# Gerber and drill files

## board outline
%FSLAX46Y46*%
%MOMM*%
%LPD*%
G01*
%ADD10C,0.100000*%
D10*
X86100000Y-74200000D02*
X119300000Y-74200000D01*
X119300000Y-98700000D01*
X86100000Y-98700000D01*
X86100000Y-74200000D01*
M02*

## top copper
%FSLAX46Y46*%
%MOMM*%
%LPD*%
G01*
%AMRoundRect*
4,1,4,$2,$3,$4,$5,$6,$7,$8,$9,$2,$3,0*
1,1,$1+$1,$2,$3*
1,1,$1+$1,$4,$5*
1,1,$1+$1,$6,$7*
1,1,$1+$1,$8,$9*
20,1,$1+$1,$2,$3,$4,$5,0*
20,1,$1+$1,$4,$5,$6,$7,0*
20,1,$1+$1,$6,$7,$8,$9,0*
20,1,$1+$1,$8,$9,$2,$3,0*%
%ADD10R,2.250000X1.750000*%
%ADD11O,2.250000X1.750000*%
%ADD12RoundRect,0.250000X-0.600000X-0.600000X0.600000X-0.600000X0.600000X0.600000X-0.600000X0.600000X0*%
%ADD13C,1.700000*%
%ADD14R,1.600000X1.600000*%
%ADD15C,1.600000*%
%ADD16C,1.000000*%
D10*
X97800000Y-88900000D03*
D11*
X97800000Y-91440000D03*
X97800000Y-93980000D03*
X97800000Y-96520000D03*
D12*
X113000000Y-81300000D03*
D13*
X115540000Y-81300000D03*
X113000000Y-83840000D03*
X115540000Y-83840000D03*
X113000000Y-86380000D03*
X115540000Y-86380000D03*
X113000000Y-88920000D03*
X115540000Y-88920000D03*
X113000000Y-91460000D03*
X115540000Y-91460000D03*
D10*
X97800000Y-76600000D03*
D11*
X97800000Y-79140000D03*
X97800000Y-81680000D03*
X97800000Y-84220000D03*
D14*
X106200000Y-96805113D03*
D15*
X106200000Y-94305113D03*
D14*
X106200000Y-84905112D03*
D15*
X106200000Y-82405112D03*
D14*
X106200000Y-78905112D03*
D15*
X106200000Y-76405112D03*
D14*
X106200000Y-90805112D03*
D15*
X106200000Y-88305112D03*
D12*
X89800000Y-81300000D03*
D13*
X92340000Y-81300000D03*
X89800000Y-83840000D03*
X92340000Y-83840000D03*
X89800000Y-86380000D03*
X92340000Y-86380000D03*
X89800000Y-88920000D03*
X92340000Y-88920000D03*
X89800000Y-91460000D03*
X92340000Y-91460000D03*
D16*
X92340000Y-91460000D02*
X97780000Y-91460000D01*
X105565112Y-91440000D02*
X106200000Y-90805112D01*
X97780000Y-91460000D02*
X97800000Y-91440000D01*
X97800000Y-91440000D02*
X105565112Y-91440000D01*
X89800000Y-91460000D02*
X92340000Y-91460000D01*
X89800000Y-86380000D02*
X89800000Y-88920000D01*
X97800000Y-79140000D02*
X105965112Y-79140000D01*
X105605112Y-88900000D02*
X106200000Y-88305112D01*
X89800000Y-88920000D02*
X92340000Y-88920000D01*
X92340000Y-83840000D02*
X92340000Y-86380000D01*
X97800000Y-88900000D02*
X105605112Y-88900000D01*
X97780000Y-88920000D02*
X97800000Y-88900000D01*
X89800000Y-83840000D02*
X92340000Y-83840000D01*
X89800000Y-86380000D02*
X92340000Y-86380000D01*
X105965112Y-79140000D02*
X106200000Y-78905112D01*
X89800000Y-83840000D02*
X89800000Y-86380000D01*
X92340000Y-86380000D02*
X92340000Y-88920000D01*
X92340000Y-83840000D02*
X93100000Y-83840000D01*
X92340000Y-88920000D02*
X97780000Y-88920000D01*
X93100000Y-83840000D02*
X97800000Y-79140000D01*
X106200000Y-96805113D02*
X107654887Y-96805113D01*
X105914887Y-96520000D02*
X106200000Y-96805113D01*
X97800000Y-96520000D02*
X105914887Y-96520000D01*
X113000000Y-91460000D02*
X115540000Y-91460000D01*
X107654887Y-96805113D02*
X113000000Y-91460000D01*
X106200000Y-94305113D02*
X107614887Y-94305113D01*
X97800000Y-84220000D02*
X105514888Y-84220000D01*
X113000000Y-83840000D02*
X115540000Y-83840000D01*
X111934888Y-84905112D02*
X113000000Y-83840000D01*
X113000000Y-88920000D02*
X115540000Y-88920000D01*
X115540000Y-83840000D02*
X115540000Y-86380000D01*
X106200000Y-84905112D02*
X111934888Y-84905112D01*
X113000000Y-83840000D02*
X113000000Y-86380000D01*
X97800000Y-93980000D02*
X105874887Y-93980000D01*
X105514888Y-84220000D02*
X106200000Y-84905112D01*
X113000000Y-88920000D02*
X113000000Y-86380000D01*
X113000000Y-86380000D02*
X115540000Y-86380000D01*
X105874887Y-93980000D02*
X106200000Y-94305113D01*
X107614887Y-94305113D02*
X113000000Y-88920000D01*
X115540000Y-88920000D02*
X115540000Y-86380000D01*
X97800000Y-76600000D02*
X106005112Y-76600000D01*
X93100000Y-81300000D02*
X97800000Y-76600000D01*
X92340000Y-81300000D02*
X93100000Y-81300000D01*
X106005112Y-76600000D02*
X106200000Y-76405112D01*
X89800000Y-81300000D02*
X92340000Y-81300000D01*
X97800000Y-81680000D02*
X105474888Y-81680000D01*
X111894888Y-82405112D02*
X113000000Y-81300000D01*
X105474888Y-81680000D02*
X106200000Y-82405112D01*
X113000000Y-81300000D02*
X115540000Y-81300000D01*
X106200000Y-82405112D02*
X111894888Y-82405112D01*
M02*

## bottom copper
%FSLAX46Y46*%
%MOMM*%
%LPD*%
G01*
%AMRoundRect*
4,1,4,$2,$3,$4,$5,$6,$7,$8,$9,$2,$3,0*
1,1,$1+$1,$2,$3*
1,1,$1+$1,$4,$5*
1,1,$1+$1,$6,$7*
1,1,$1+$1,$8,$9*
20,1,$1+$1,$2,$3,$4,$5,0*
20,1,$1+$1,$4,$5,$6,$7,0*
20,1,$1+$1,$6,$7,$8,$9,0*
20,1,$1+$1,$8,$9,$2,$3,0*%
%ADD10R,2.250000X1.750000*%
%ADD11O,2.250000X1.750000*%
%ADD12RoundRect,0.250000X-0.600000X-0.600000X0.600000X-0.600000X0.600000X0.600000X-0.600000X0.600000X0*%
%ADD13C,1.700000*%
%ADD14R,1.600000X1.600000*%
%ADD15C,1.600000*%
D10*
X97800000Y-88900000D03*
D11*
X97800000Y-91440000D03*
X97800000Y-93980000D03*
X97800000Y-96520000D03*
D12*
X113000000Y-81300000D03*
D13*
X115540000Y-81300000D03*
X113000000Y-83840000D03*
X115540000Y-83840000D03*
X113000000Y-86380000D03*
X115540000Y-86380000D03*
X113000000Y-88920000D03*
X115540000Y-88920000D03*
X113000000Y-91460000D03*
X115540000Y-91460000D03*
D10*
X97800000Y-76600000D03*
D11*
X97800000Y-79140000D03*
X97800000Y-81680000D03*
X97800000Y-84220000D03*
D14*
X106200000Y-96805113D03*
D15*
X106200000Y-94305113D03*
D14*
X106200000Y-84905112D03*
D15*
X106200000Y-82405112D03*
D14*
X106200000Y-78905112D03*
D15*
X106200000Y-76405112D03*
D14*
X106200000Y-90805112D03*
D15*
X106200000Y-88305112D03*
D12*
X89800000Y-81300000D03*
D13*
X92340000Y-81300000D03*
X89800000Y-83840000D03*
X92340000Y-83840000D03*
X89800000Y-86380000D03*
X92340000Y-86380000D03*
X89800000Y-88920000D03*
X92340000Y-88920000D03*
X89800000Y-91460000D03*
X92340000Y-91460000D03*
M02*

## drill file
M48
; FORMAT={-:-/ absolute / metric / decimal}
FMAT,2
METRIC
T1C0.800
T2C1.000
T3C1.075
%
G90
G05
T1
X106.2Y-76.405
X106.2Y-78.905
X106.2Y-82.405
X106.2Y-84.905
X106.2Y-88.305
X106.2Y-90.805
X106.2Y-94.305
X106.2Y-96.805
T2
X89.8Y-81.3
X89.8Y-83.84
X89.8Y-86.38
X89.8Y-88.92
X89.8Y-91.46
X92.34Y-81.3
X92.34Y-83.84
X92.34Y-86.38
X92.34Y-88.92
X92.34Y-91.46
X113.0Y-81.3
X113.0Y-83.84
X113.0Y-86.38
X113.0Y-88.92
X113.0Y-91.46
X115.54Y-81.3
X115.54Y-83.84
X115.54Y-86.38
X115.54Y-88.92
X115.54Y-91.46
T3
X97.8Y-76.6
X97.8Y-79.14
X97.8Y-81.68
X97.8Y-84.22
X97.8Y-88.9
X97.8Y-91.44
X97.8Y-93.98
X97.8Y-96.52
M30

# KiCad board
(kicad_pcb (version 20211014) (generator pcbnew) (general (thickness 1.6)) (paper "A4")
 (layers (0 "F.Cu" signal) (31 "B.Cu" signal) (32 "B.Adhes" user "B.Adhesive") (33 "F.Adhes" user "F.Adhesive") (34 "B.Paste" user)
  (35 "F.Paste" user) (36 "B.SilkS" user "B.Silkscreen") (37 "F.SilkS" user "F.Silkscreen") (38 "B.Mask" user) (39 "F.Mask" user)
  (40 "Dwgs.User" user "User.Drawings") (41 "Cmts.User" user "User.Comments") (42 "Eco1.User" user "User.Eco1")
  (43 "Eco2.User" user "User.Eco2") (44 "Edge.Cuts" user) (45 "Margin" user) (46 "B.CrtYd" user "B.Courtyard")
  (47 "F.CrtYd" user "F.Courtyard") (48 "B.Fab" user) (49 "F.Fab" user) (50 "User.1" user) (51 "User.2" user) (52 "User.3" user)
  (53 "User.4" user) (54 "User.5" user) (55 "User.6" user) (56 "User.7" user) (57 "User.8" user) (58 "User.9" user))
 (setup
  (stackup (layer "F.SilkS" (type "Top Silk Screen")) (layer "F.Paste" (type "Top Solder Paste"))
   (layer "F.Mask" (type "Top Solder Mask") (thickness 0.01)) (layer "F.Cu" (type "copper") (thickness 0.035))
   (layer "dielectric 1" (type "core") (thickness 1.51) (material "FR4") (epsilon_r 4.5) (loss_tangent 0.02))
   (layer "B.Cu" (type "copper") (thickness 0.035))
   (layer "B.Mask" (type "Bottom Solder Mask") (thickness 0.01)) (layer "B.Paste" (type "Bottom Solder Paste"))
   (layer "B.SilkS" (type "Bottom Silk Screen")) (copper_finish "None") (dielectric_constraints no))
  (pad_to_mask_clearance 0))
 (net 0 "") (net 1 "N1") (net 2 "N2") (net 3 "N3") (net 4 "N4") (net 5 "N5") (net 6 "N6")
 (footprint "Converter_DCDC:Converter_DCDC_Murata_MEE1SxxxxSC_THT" (layer "F.Cu") (at 97.8 88.9)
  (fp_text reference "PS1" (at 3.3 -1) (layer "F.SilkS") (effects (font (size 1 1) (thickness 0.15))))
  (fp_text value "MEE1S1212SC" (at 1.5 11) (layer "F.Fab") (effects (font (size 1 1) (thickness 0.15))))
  (pad "1" thru_hole rect locked (at 0 0 270) (size 1.75 2.25) (drill 1.075) (layers *.Cu *.Mask) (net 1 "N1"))
  (pad "2" thru_hole oval locked (at 0 2.54 270) (size 1.75 2.25) (drill 1.075) (layers *.Cu *.Mask) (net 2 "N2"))
  (pad "3" thru_hole oval locked (at 0 5.08 270) (size 1.75 2.25) (drill 1.075) (layers *.Cu *.Mask) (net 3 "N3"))
  (pad "4" thru_hole oval locked (at 0 7.62 270) (size 1.75 2.25) (drill 1.075) (layers *.Cu *.Mask) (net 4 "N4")))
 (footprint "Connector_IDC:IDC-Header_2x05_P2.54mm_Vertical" (layer "F.Cu") (at 113 81.3)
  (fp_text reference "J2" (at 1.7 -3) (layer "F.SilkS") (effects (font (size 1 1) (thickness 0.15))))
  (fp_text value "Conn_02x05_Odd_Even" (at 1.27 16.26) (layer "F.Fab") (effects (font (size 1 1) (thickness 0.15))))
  (pad "1" thru_hole roundrect locked (at 0 0) (size 1.7 1.7) (drill 1) (layers *.Cu *.Mask) (roundrect_rratio 0.147059) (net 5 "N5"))
  (pad "2" thru_hole circle locked (at 2.54 0) (size 1.7 1.7) (drill 1) (layers *.Cu *.Mask) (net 5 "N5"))
  (pad "3" thru_hole circle locked (at 0 2.54) (size 1.7 1.7) (drill 1) (layers *.Cu *.Mask) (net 3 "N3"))
  (pad "4" thru_hole circle locked (at 2.54 2.54) (size 1.7 1.7) (drill 1) (layers *.Cu *.Mask) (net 3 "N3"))
  (pad "5" thru_hole circle locked (at 0 5.08) (size 1.7 1.7) (drill 1) (layers *.Cu *.Mask) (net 3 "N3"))
  (pad "6" thru_hole circle locked (at 2.54 5.08) (size 1.7 1.7) (drill 1) (layers *.Cu *.Mask) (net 3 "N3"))
  (pad "7" thru_hole circle locked (at 0 7.62) (size 1.7 1.7) (drill 1) (layers *.Cu *.Mask) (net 3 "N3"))
  (pad "8" thru_hole circle locked (at 2.54 7.62) (size 1.7 1.7) (drill 1) (layers *.Cu *.Mask) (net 3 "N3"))
  (pad "9" thru_hole circle locked (at 0 10.16) (size 1.7 1.7) (drill 1) (layers *.Cu *.Mask) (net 4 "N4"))
  (pad "10" thru_hole circle locked (at 2.54 10.16) (size 1.7 1.7) (drill 1) (layers *.Cu *.Mask) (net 4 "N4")))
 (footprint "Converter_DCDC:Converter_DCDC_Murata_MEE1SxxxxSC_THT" (layer "F.Cu") (at 97.8 76.6)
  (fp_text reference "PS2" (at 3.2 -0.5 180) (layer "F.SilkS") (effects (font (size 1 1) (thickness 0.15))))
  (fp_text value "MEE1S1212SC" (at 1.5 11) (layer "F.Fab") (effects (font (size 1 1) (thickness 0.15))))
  (pad "1" thru_hole rect locked (at 0 0 270) (size 1.75 2.25) (drill 1.075) (layers *.Cu *.Mask) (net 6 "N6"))
  (pad "2" thru_hole oval locked (at 0 2.54 270) (size 1.75 2.25) (drill 1.075) (layers *.Cu *.Mask) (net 1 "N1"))
  (pad "3" thru_hole oval locked (at 0 5.08 270) (size 1.75 2.25) (drill 1.075) (layers *.Cu *.Mask) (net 5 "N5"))
  (pad "4" thru_hole oval locked (at 0 7.62 270) (size 1.75 2.25) (drill 1.075) (layers *.Cu *.Mask) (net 3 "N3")))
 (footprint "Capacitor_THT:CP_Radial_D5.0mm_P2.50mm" (layer "F.Cu") (at 106.2 96.805113 90)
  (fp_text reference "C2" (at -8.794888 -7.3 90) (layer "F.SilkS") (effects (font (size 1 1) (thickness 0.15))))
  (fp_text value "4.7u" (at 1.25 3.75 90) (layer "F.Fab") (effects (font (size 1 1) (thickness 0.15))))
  (pad "1" thru_hole rect locked (at 0 0 90) (size 1.6 1.6) (drill 0.8) (layers *.Cu *.Mask) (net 4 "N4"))
  (pad "2" thru_hole circle locked (at 2.5 0 90) (size 1.6 1.6) (drill 0.8) (layers *.Cu *.Mask) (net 3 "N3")))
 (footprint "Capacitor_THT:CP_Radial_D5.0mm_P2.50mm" (layer "F.Cu") (at 106.2 84.905112 90)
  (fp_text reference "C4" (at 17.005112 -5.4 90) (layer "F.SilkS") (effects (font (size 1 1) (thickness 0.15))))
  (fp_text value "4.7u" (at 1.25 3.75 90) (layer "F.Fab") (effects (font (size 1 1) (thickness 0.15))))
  (pad "1" thru_hole rect locked (at 0 0 90) (size 1.6 1.6) (drill 0.8) (layers *.Cu *.Mask) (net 3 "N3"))
  (pad "2" thru_hole circle locked (at 2.5 0 90) (size 1.6 1.6) (drill 0.8) (layers *.Cu *.Mask) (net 5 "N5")))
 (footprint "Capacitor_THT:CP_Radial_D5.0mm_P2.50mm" (layer "F.Cu") (at 106.2 78.905112 90)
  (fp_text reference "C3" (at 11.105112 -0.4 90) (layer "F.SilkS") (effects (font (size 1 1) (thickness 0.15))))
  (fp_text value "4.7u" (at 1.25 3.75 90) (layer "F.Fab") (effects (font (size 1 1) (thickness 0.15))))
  (pad "1" thru_hole rect locked (at 0 0 90) (size 1.6 1.6) (drill 0.8) (layers *.Cu *.Mask) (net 1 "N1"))
  (pad "2" thru_hole circle locked (at 2.5 0 90) (size 1.6 1.6) (drill 0.8) (layers *.Cu *.Mask) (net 6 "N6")))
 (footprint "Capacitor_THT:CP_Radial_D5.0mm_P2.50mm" (layer "F.Cu") (at 106.2 90.805112 90)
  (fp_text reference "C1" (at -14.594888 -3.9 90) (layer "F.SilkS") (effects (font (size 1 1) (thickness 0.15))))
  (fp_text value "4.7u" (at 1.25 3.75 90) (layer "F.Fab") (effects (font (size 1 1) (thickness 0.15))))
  (pad "1" thru_hole rect locked (at 0 0 90) (size 1.6 1.6) (drill 0.8) (layers *.Cu *.Mask) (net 2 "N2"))
  (pad "2" thru_hole circle locked (at 2.5 0 90) (size 1.6 1.6) (drill 0.8) (layers *.Cu *.Mask) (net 1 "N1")))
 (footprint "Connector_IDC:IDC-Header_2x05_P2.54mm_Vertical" (layer "F.Cu") (at 89.8 81.3)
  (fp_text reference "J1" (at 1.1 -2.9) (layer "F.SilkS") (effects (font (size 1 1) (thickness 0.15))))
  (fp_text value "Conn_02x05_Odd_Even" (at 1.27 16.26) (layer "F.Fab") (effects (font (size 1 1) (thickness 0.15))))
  (pad "1" thru_hole roundrect locked (at 0 0) (size 1.7 1.7) (drill 1) (layers *.Cu *.Mask) (roundrect_rratio 0.147059) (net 6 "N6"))
  (pad "2" thru_hole circle locked (at 2.54 0) (size 1.7 1.7) (drill 1) (layers *.Cu *.Mask) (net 6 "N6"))
  (pad "3" thru_hole circle locked (at 0 2.54) (size 1.7 1.7) (drill 1) (layers *.Cu *.Mask) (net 1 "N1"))
  (pad "4" thru_hole circle locked (at 2.54 2.54) (size 1.7 1.7) (drill 1) (layers *.Cu *.Mask) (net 1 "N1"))
  (pad "5" thru_hole circle locked (at 0 5.08) (size 1.7 1.7) (drill 1) (layers *.Cu *.Mask) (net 1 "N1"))
  (pad "6" thru_hole circle locked (at 2.54 5.08) (size 1.7 1.7) (drill 1) (layers *.Cu *.Mask) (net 1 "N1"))
  (pad "7" thru_hole circle locked (at 0 7.62) (size 1.7 1.7) (drill 1) (layers *.Cu *.Mask) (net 1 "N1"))
  (pad "8" thru_hole circle locked (at 2.54 7.62) (size 1.7 1.7) (drill 1) (layers *.Cu *.Mask) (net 1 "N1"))
  (pad "9" thru_hole circle locked (at 0 10.16) (size 1.7 1.7) (drill 1) (layers *.Cu *.Mask) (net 2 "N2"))
  (pad "10" thru_hole circle locked (at 2.54 10.16) (size 1.7 1.7) (drill 1) (layers *.Cu *.Mask) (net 2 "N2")))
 (gr_rect (start 86.1 74.2) (end 119.3 98.7) (layer "Edge.Cuts") (width 0.1) (fill none))
 (segment (start 92.34 91.46) (end 97.78 91.46) (width 1) (layer "F.Cu") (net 2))
 (segment (start 105.565112 91.44) (end 106.2 90.805112) (width 1) (layer "F.Cu") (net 2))
 (segment (start 97.78 91.46) (end 97.8 91.44) (width 1) (layer "F.Cu") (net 2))
 (segment (start 97.8 91.44) (end 105.565112 91.44) (width 1) (layer "F.Cu") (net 2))
 (segment (start 89.8 91.46) (end 92.34 91.46) (width 1) (layer "F.Cu") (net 2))
 (segment (start 89.8 86.38) (end 89.8 88.92) (width 1) (layer "F.Cu") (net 1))
 (segment (start 97.8 79.14) (end 105.965112 79.14) (width 1) (layer "F.Cu") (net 1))
 (segment (start 105.605112 88.9) (end 106.2 88.305112) (width 1) (layer "F.Cu") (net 1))
 (segment (start 89.8 88.92) (end 92.34 88.92) (width 1) (layer "F.Cu") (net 1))
 (segment (start 92.34 83.84) (end 92.34 86.38) (width 1) (layer "F.Cu") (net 1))
 (segment (start 97.8 88.9) (end 105.605112 88.9) (width 1) (layer "F.Cu") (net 1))
 (segment (start 97.78 88.92) (end 97.8 88.9) (width 1) (layer "F.Cu") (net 1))
 (segment (start 89.8 83.84) (end 92.34 83.84) (width 1) (layer "F.Cu") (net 1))
 (segment (start 89.8 86.38) (end 92.34 86.38) (width 1) (layer "F.Cu") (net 1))
 (segment (start 105.965112 79.14) (end 106.2 78.905112) (width 1) (layer "F.Cu") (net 1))
 (segment (start 89.8 83.84) (end 89.8 86.38) (width 1) (layer "F.Cu") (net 1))
 (segment (start 92.34 86.38) (end 92.34 88.92) (width 1) (layer "F.Cu") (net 1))
 (segment (start 92.34 83.84) (end 93.1 83.84) (width 1) (layer "F.Cu") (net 1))
 (segment (start 92.34 88.92) (end 97.78 88.92) (width 1) (layer "F.Cu") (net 1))
 (segment (start 93.1 83.84) (end 97.8 79.14) (width 1) (layer "F.Cu") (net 1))
 (segment (start 106.2 96.805113) (end 107.654887 96.805113) (width 1) (layer "F.Cu") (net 4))
 (segment (start 105.914887 96.52) (end 106.2 96.805113) (width 1) (layer "F.Cu") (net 4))
 (segment (start 97.8 96.52) (end 105.914887 96.52) (width 1) (layer "F.Cu") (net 4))
 (segment (start 113 91.46) (end 115.54 91.46) (width 1) (layer "F.Cu") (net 4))
 (segment (start 107.654887 96.805113) (end 113 91.46) (width 1) (layer "F.Cu") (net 4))
 (segment (start 106.2 94.305113) (end 107.614887 94.305113) (width 1) (layer "F.Cu") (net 3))
 (segment (start 97.8 84.22) (end 105.514888 84.22) (width 1) (layer "F.Cu") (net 3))
 (segment (start 113 83.84) (end 115.54 83.84) (width 1) (layer "F.Cu") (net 3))
 (segment (start 111.934888 84.905112) (end 113 83.84) (width 1) (layer "F.Cu") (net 3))
 (segment (start 113 88.92) (end 115.54 88.92) (width 1) (layer "F.Cu") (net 3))
 (segment (start 115.54 83.84) (end 115.54 86.38) (width 1) (layer "F.Cu") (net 3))
 (segment (start 106.2 84.905112) (end 111.934888 84.905112) (width 1) (layer "F.Cu") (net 3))
 (segment (start 113 83.84) (end 113 86.38) (width 1) (layer "F.Cu") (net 3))
 (segment (start 97.8 93.98) (end 105.874887 93.98) (width 1) (layer "F.Cu") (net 3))
 (segment (start 105.514888 84.22) (end 106.2 84.905112) (width 1) (layer "F.Cu") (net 3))
 (segment (start 113 88.92) (end 113 86.38) (width 1) (layer "F.Cu") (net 3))
 (segment (start 113 86.38) (end 115.54 86.38) (width 1) (layer "F.Cu") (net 3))
 (segment (start 105.874887 93.98) (end 106.2 94.305113) (width 1) (layer "F.Cu") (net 3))
 (segment (start 107.614887 94.305113) (end 113 88.92) (width 1) (layer "F.Cu") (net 3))
 (segment (start 115.54 88.92) (end 115.54 86.38) (width 1) (layer "F.Cu") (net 3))
 (segment (start 97.8 76.6) (end 106.005112 76.6) (width 1) (layer "F.Cu") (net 6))
 (segment (start 93.1 81.3) (end 97.8 76.6) (width 1) (layer "F.Cu") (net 6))
 (segment (start 92.34 81.3) (end 93.1 81.3) (width 1) (layer "F.Cu") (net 6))
 (segment (start 106.005112 76.6) (end 106.2 76.405112) (width 1) (layer "F.Cu") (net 6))
 (segment (start 89.8 81.3) (end 92.34 81.3) (width 1) (layer "F.Cu") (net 6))
 (segment (start 97.8 81.68) (end 105.474888 81.68) (width 1) (layer "F.Cu") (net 5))
 (segment (start 111.894888 82.405112) (end 113 81.3) (width 1) (layer "F.Cu") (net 5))
 (segment (start 105.474888 81.68) (end 106.2 82.405112) (width 1) (layer "F.Cu") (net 5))
 (segment (start 113 81.3) (end 115.54 81.3) (width 1) (layer "F.Cu") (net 5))
 (segment (start 106.2 82.405112) (end 111.894888 82.405112) (width 1) (layer "F.Cu") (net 5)))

